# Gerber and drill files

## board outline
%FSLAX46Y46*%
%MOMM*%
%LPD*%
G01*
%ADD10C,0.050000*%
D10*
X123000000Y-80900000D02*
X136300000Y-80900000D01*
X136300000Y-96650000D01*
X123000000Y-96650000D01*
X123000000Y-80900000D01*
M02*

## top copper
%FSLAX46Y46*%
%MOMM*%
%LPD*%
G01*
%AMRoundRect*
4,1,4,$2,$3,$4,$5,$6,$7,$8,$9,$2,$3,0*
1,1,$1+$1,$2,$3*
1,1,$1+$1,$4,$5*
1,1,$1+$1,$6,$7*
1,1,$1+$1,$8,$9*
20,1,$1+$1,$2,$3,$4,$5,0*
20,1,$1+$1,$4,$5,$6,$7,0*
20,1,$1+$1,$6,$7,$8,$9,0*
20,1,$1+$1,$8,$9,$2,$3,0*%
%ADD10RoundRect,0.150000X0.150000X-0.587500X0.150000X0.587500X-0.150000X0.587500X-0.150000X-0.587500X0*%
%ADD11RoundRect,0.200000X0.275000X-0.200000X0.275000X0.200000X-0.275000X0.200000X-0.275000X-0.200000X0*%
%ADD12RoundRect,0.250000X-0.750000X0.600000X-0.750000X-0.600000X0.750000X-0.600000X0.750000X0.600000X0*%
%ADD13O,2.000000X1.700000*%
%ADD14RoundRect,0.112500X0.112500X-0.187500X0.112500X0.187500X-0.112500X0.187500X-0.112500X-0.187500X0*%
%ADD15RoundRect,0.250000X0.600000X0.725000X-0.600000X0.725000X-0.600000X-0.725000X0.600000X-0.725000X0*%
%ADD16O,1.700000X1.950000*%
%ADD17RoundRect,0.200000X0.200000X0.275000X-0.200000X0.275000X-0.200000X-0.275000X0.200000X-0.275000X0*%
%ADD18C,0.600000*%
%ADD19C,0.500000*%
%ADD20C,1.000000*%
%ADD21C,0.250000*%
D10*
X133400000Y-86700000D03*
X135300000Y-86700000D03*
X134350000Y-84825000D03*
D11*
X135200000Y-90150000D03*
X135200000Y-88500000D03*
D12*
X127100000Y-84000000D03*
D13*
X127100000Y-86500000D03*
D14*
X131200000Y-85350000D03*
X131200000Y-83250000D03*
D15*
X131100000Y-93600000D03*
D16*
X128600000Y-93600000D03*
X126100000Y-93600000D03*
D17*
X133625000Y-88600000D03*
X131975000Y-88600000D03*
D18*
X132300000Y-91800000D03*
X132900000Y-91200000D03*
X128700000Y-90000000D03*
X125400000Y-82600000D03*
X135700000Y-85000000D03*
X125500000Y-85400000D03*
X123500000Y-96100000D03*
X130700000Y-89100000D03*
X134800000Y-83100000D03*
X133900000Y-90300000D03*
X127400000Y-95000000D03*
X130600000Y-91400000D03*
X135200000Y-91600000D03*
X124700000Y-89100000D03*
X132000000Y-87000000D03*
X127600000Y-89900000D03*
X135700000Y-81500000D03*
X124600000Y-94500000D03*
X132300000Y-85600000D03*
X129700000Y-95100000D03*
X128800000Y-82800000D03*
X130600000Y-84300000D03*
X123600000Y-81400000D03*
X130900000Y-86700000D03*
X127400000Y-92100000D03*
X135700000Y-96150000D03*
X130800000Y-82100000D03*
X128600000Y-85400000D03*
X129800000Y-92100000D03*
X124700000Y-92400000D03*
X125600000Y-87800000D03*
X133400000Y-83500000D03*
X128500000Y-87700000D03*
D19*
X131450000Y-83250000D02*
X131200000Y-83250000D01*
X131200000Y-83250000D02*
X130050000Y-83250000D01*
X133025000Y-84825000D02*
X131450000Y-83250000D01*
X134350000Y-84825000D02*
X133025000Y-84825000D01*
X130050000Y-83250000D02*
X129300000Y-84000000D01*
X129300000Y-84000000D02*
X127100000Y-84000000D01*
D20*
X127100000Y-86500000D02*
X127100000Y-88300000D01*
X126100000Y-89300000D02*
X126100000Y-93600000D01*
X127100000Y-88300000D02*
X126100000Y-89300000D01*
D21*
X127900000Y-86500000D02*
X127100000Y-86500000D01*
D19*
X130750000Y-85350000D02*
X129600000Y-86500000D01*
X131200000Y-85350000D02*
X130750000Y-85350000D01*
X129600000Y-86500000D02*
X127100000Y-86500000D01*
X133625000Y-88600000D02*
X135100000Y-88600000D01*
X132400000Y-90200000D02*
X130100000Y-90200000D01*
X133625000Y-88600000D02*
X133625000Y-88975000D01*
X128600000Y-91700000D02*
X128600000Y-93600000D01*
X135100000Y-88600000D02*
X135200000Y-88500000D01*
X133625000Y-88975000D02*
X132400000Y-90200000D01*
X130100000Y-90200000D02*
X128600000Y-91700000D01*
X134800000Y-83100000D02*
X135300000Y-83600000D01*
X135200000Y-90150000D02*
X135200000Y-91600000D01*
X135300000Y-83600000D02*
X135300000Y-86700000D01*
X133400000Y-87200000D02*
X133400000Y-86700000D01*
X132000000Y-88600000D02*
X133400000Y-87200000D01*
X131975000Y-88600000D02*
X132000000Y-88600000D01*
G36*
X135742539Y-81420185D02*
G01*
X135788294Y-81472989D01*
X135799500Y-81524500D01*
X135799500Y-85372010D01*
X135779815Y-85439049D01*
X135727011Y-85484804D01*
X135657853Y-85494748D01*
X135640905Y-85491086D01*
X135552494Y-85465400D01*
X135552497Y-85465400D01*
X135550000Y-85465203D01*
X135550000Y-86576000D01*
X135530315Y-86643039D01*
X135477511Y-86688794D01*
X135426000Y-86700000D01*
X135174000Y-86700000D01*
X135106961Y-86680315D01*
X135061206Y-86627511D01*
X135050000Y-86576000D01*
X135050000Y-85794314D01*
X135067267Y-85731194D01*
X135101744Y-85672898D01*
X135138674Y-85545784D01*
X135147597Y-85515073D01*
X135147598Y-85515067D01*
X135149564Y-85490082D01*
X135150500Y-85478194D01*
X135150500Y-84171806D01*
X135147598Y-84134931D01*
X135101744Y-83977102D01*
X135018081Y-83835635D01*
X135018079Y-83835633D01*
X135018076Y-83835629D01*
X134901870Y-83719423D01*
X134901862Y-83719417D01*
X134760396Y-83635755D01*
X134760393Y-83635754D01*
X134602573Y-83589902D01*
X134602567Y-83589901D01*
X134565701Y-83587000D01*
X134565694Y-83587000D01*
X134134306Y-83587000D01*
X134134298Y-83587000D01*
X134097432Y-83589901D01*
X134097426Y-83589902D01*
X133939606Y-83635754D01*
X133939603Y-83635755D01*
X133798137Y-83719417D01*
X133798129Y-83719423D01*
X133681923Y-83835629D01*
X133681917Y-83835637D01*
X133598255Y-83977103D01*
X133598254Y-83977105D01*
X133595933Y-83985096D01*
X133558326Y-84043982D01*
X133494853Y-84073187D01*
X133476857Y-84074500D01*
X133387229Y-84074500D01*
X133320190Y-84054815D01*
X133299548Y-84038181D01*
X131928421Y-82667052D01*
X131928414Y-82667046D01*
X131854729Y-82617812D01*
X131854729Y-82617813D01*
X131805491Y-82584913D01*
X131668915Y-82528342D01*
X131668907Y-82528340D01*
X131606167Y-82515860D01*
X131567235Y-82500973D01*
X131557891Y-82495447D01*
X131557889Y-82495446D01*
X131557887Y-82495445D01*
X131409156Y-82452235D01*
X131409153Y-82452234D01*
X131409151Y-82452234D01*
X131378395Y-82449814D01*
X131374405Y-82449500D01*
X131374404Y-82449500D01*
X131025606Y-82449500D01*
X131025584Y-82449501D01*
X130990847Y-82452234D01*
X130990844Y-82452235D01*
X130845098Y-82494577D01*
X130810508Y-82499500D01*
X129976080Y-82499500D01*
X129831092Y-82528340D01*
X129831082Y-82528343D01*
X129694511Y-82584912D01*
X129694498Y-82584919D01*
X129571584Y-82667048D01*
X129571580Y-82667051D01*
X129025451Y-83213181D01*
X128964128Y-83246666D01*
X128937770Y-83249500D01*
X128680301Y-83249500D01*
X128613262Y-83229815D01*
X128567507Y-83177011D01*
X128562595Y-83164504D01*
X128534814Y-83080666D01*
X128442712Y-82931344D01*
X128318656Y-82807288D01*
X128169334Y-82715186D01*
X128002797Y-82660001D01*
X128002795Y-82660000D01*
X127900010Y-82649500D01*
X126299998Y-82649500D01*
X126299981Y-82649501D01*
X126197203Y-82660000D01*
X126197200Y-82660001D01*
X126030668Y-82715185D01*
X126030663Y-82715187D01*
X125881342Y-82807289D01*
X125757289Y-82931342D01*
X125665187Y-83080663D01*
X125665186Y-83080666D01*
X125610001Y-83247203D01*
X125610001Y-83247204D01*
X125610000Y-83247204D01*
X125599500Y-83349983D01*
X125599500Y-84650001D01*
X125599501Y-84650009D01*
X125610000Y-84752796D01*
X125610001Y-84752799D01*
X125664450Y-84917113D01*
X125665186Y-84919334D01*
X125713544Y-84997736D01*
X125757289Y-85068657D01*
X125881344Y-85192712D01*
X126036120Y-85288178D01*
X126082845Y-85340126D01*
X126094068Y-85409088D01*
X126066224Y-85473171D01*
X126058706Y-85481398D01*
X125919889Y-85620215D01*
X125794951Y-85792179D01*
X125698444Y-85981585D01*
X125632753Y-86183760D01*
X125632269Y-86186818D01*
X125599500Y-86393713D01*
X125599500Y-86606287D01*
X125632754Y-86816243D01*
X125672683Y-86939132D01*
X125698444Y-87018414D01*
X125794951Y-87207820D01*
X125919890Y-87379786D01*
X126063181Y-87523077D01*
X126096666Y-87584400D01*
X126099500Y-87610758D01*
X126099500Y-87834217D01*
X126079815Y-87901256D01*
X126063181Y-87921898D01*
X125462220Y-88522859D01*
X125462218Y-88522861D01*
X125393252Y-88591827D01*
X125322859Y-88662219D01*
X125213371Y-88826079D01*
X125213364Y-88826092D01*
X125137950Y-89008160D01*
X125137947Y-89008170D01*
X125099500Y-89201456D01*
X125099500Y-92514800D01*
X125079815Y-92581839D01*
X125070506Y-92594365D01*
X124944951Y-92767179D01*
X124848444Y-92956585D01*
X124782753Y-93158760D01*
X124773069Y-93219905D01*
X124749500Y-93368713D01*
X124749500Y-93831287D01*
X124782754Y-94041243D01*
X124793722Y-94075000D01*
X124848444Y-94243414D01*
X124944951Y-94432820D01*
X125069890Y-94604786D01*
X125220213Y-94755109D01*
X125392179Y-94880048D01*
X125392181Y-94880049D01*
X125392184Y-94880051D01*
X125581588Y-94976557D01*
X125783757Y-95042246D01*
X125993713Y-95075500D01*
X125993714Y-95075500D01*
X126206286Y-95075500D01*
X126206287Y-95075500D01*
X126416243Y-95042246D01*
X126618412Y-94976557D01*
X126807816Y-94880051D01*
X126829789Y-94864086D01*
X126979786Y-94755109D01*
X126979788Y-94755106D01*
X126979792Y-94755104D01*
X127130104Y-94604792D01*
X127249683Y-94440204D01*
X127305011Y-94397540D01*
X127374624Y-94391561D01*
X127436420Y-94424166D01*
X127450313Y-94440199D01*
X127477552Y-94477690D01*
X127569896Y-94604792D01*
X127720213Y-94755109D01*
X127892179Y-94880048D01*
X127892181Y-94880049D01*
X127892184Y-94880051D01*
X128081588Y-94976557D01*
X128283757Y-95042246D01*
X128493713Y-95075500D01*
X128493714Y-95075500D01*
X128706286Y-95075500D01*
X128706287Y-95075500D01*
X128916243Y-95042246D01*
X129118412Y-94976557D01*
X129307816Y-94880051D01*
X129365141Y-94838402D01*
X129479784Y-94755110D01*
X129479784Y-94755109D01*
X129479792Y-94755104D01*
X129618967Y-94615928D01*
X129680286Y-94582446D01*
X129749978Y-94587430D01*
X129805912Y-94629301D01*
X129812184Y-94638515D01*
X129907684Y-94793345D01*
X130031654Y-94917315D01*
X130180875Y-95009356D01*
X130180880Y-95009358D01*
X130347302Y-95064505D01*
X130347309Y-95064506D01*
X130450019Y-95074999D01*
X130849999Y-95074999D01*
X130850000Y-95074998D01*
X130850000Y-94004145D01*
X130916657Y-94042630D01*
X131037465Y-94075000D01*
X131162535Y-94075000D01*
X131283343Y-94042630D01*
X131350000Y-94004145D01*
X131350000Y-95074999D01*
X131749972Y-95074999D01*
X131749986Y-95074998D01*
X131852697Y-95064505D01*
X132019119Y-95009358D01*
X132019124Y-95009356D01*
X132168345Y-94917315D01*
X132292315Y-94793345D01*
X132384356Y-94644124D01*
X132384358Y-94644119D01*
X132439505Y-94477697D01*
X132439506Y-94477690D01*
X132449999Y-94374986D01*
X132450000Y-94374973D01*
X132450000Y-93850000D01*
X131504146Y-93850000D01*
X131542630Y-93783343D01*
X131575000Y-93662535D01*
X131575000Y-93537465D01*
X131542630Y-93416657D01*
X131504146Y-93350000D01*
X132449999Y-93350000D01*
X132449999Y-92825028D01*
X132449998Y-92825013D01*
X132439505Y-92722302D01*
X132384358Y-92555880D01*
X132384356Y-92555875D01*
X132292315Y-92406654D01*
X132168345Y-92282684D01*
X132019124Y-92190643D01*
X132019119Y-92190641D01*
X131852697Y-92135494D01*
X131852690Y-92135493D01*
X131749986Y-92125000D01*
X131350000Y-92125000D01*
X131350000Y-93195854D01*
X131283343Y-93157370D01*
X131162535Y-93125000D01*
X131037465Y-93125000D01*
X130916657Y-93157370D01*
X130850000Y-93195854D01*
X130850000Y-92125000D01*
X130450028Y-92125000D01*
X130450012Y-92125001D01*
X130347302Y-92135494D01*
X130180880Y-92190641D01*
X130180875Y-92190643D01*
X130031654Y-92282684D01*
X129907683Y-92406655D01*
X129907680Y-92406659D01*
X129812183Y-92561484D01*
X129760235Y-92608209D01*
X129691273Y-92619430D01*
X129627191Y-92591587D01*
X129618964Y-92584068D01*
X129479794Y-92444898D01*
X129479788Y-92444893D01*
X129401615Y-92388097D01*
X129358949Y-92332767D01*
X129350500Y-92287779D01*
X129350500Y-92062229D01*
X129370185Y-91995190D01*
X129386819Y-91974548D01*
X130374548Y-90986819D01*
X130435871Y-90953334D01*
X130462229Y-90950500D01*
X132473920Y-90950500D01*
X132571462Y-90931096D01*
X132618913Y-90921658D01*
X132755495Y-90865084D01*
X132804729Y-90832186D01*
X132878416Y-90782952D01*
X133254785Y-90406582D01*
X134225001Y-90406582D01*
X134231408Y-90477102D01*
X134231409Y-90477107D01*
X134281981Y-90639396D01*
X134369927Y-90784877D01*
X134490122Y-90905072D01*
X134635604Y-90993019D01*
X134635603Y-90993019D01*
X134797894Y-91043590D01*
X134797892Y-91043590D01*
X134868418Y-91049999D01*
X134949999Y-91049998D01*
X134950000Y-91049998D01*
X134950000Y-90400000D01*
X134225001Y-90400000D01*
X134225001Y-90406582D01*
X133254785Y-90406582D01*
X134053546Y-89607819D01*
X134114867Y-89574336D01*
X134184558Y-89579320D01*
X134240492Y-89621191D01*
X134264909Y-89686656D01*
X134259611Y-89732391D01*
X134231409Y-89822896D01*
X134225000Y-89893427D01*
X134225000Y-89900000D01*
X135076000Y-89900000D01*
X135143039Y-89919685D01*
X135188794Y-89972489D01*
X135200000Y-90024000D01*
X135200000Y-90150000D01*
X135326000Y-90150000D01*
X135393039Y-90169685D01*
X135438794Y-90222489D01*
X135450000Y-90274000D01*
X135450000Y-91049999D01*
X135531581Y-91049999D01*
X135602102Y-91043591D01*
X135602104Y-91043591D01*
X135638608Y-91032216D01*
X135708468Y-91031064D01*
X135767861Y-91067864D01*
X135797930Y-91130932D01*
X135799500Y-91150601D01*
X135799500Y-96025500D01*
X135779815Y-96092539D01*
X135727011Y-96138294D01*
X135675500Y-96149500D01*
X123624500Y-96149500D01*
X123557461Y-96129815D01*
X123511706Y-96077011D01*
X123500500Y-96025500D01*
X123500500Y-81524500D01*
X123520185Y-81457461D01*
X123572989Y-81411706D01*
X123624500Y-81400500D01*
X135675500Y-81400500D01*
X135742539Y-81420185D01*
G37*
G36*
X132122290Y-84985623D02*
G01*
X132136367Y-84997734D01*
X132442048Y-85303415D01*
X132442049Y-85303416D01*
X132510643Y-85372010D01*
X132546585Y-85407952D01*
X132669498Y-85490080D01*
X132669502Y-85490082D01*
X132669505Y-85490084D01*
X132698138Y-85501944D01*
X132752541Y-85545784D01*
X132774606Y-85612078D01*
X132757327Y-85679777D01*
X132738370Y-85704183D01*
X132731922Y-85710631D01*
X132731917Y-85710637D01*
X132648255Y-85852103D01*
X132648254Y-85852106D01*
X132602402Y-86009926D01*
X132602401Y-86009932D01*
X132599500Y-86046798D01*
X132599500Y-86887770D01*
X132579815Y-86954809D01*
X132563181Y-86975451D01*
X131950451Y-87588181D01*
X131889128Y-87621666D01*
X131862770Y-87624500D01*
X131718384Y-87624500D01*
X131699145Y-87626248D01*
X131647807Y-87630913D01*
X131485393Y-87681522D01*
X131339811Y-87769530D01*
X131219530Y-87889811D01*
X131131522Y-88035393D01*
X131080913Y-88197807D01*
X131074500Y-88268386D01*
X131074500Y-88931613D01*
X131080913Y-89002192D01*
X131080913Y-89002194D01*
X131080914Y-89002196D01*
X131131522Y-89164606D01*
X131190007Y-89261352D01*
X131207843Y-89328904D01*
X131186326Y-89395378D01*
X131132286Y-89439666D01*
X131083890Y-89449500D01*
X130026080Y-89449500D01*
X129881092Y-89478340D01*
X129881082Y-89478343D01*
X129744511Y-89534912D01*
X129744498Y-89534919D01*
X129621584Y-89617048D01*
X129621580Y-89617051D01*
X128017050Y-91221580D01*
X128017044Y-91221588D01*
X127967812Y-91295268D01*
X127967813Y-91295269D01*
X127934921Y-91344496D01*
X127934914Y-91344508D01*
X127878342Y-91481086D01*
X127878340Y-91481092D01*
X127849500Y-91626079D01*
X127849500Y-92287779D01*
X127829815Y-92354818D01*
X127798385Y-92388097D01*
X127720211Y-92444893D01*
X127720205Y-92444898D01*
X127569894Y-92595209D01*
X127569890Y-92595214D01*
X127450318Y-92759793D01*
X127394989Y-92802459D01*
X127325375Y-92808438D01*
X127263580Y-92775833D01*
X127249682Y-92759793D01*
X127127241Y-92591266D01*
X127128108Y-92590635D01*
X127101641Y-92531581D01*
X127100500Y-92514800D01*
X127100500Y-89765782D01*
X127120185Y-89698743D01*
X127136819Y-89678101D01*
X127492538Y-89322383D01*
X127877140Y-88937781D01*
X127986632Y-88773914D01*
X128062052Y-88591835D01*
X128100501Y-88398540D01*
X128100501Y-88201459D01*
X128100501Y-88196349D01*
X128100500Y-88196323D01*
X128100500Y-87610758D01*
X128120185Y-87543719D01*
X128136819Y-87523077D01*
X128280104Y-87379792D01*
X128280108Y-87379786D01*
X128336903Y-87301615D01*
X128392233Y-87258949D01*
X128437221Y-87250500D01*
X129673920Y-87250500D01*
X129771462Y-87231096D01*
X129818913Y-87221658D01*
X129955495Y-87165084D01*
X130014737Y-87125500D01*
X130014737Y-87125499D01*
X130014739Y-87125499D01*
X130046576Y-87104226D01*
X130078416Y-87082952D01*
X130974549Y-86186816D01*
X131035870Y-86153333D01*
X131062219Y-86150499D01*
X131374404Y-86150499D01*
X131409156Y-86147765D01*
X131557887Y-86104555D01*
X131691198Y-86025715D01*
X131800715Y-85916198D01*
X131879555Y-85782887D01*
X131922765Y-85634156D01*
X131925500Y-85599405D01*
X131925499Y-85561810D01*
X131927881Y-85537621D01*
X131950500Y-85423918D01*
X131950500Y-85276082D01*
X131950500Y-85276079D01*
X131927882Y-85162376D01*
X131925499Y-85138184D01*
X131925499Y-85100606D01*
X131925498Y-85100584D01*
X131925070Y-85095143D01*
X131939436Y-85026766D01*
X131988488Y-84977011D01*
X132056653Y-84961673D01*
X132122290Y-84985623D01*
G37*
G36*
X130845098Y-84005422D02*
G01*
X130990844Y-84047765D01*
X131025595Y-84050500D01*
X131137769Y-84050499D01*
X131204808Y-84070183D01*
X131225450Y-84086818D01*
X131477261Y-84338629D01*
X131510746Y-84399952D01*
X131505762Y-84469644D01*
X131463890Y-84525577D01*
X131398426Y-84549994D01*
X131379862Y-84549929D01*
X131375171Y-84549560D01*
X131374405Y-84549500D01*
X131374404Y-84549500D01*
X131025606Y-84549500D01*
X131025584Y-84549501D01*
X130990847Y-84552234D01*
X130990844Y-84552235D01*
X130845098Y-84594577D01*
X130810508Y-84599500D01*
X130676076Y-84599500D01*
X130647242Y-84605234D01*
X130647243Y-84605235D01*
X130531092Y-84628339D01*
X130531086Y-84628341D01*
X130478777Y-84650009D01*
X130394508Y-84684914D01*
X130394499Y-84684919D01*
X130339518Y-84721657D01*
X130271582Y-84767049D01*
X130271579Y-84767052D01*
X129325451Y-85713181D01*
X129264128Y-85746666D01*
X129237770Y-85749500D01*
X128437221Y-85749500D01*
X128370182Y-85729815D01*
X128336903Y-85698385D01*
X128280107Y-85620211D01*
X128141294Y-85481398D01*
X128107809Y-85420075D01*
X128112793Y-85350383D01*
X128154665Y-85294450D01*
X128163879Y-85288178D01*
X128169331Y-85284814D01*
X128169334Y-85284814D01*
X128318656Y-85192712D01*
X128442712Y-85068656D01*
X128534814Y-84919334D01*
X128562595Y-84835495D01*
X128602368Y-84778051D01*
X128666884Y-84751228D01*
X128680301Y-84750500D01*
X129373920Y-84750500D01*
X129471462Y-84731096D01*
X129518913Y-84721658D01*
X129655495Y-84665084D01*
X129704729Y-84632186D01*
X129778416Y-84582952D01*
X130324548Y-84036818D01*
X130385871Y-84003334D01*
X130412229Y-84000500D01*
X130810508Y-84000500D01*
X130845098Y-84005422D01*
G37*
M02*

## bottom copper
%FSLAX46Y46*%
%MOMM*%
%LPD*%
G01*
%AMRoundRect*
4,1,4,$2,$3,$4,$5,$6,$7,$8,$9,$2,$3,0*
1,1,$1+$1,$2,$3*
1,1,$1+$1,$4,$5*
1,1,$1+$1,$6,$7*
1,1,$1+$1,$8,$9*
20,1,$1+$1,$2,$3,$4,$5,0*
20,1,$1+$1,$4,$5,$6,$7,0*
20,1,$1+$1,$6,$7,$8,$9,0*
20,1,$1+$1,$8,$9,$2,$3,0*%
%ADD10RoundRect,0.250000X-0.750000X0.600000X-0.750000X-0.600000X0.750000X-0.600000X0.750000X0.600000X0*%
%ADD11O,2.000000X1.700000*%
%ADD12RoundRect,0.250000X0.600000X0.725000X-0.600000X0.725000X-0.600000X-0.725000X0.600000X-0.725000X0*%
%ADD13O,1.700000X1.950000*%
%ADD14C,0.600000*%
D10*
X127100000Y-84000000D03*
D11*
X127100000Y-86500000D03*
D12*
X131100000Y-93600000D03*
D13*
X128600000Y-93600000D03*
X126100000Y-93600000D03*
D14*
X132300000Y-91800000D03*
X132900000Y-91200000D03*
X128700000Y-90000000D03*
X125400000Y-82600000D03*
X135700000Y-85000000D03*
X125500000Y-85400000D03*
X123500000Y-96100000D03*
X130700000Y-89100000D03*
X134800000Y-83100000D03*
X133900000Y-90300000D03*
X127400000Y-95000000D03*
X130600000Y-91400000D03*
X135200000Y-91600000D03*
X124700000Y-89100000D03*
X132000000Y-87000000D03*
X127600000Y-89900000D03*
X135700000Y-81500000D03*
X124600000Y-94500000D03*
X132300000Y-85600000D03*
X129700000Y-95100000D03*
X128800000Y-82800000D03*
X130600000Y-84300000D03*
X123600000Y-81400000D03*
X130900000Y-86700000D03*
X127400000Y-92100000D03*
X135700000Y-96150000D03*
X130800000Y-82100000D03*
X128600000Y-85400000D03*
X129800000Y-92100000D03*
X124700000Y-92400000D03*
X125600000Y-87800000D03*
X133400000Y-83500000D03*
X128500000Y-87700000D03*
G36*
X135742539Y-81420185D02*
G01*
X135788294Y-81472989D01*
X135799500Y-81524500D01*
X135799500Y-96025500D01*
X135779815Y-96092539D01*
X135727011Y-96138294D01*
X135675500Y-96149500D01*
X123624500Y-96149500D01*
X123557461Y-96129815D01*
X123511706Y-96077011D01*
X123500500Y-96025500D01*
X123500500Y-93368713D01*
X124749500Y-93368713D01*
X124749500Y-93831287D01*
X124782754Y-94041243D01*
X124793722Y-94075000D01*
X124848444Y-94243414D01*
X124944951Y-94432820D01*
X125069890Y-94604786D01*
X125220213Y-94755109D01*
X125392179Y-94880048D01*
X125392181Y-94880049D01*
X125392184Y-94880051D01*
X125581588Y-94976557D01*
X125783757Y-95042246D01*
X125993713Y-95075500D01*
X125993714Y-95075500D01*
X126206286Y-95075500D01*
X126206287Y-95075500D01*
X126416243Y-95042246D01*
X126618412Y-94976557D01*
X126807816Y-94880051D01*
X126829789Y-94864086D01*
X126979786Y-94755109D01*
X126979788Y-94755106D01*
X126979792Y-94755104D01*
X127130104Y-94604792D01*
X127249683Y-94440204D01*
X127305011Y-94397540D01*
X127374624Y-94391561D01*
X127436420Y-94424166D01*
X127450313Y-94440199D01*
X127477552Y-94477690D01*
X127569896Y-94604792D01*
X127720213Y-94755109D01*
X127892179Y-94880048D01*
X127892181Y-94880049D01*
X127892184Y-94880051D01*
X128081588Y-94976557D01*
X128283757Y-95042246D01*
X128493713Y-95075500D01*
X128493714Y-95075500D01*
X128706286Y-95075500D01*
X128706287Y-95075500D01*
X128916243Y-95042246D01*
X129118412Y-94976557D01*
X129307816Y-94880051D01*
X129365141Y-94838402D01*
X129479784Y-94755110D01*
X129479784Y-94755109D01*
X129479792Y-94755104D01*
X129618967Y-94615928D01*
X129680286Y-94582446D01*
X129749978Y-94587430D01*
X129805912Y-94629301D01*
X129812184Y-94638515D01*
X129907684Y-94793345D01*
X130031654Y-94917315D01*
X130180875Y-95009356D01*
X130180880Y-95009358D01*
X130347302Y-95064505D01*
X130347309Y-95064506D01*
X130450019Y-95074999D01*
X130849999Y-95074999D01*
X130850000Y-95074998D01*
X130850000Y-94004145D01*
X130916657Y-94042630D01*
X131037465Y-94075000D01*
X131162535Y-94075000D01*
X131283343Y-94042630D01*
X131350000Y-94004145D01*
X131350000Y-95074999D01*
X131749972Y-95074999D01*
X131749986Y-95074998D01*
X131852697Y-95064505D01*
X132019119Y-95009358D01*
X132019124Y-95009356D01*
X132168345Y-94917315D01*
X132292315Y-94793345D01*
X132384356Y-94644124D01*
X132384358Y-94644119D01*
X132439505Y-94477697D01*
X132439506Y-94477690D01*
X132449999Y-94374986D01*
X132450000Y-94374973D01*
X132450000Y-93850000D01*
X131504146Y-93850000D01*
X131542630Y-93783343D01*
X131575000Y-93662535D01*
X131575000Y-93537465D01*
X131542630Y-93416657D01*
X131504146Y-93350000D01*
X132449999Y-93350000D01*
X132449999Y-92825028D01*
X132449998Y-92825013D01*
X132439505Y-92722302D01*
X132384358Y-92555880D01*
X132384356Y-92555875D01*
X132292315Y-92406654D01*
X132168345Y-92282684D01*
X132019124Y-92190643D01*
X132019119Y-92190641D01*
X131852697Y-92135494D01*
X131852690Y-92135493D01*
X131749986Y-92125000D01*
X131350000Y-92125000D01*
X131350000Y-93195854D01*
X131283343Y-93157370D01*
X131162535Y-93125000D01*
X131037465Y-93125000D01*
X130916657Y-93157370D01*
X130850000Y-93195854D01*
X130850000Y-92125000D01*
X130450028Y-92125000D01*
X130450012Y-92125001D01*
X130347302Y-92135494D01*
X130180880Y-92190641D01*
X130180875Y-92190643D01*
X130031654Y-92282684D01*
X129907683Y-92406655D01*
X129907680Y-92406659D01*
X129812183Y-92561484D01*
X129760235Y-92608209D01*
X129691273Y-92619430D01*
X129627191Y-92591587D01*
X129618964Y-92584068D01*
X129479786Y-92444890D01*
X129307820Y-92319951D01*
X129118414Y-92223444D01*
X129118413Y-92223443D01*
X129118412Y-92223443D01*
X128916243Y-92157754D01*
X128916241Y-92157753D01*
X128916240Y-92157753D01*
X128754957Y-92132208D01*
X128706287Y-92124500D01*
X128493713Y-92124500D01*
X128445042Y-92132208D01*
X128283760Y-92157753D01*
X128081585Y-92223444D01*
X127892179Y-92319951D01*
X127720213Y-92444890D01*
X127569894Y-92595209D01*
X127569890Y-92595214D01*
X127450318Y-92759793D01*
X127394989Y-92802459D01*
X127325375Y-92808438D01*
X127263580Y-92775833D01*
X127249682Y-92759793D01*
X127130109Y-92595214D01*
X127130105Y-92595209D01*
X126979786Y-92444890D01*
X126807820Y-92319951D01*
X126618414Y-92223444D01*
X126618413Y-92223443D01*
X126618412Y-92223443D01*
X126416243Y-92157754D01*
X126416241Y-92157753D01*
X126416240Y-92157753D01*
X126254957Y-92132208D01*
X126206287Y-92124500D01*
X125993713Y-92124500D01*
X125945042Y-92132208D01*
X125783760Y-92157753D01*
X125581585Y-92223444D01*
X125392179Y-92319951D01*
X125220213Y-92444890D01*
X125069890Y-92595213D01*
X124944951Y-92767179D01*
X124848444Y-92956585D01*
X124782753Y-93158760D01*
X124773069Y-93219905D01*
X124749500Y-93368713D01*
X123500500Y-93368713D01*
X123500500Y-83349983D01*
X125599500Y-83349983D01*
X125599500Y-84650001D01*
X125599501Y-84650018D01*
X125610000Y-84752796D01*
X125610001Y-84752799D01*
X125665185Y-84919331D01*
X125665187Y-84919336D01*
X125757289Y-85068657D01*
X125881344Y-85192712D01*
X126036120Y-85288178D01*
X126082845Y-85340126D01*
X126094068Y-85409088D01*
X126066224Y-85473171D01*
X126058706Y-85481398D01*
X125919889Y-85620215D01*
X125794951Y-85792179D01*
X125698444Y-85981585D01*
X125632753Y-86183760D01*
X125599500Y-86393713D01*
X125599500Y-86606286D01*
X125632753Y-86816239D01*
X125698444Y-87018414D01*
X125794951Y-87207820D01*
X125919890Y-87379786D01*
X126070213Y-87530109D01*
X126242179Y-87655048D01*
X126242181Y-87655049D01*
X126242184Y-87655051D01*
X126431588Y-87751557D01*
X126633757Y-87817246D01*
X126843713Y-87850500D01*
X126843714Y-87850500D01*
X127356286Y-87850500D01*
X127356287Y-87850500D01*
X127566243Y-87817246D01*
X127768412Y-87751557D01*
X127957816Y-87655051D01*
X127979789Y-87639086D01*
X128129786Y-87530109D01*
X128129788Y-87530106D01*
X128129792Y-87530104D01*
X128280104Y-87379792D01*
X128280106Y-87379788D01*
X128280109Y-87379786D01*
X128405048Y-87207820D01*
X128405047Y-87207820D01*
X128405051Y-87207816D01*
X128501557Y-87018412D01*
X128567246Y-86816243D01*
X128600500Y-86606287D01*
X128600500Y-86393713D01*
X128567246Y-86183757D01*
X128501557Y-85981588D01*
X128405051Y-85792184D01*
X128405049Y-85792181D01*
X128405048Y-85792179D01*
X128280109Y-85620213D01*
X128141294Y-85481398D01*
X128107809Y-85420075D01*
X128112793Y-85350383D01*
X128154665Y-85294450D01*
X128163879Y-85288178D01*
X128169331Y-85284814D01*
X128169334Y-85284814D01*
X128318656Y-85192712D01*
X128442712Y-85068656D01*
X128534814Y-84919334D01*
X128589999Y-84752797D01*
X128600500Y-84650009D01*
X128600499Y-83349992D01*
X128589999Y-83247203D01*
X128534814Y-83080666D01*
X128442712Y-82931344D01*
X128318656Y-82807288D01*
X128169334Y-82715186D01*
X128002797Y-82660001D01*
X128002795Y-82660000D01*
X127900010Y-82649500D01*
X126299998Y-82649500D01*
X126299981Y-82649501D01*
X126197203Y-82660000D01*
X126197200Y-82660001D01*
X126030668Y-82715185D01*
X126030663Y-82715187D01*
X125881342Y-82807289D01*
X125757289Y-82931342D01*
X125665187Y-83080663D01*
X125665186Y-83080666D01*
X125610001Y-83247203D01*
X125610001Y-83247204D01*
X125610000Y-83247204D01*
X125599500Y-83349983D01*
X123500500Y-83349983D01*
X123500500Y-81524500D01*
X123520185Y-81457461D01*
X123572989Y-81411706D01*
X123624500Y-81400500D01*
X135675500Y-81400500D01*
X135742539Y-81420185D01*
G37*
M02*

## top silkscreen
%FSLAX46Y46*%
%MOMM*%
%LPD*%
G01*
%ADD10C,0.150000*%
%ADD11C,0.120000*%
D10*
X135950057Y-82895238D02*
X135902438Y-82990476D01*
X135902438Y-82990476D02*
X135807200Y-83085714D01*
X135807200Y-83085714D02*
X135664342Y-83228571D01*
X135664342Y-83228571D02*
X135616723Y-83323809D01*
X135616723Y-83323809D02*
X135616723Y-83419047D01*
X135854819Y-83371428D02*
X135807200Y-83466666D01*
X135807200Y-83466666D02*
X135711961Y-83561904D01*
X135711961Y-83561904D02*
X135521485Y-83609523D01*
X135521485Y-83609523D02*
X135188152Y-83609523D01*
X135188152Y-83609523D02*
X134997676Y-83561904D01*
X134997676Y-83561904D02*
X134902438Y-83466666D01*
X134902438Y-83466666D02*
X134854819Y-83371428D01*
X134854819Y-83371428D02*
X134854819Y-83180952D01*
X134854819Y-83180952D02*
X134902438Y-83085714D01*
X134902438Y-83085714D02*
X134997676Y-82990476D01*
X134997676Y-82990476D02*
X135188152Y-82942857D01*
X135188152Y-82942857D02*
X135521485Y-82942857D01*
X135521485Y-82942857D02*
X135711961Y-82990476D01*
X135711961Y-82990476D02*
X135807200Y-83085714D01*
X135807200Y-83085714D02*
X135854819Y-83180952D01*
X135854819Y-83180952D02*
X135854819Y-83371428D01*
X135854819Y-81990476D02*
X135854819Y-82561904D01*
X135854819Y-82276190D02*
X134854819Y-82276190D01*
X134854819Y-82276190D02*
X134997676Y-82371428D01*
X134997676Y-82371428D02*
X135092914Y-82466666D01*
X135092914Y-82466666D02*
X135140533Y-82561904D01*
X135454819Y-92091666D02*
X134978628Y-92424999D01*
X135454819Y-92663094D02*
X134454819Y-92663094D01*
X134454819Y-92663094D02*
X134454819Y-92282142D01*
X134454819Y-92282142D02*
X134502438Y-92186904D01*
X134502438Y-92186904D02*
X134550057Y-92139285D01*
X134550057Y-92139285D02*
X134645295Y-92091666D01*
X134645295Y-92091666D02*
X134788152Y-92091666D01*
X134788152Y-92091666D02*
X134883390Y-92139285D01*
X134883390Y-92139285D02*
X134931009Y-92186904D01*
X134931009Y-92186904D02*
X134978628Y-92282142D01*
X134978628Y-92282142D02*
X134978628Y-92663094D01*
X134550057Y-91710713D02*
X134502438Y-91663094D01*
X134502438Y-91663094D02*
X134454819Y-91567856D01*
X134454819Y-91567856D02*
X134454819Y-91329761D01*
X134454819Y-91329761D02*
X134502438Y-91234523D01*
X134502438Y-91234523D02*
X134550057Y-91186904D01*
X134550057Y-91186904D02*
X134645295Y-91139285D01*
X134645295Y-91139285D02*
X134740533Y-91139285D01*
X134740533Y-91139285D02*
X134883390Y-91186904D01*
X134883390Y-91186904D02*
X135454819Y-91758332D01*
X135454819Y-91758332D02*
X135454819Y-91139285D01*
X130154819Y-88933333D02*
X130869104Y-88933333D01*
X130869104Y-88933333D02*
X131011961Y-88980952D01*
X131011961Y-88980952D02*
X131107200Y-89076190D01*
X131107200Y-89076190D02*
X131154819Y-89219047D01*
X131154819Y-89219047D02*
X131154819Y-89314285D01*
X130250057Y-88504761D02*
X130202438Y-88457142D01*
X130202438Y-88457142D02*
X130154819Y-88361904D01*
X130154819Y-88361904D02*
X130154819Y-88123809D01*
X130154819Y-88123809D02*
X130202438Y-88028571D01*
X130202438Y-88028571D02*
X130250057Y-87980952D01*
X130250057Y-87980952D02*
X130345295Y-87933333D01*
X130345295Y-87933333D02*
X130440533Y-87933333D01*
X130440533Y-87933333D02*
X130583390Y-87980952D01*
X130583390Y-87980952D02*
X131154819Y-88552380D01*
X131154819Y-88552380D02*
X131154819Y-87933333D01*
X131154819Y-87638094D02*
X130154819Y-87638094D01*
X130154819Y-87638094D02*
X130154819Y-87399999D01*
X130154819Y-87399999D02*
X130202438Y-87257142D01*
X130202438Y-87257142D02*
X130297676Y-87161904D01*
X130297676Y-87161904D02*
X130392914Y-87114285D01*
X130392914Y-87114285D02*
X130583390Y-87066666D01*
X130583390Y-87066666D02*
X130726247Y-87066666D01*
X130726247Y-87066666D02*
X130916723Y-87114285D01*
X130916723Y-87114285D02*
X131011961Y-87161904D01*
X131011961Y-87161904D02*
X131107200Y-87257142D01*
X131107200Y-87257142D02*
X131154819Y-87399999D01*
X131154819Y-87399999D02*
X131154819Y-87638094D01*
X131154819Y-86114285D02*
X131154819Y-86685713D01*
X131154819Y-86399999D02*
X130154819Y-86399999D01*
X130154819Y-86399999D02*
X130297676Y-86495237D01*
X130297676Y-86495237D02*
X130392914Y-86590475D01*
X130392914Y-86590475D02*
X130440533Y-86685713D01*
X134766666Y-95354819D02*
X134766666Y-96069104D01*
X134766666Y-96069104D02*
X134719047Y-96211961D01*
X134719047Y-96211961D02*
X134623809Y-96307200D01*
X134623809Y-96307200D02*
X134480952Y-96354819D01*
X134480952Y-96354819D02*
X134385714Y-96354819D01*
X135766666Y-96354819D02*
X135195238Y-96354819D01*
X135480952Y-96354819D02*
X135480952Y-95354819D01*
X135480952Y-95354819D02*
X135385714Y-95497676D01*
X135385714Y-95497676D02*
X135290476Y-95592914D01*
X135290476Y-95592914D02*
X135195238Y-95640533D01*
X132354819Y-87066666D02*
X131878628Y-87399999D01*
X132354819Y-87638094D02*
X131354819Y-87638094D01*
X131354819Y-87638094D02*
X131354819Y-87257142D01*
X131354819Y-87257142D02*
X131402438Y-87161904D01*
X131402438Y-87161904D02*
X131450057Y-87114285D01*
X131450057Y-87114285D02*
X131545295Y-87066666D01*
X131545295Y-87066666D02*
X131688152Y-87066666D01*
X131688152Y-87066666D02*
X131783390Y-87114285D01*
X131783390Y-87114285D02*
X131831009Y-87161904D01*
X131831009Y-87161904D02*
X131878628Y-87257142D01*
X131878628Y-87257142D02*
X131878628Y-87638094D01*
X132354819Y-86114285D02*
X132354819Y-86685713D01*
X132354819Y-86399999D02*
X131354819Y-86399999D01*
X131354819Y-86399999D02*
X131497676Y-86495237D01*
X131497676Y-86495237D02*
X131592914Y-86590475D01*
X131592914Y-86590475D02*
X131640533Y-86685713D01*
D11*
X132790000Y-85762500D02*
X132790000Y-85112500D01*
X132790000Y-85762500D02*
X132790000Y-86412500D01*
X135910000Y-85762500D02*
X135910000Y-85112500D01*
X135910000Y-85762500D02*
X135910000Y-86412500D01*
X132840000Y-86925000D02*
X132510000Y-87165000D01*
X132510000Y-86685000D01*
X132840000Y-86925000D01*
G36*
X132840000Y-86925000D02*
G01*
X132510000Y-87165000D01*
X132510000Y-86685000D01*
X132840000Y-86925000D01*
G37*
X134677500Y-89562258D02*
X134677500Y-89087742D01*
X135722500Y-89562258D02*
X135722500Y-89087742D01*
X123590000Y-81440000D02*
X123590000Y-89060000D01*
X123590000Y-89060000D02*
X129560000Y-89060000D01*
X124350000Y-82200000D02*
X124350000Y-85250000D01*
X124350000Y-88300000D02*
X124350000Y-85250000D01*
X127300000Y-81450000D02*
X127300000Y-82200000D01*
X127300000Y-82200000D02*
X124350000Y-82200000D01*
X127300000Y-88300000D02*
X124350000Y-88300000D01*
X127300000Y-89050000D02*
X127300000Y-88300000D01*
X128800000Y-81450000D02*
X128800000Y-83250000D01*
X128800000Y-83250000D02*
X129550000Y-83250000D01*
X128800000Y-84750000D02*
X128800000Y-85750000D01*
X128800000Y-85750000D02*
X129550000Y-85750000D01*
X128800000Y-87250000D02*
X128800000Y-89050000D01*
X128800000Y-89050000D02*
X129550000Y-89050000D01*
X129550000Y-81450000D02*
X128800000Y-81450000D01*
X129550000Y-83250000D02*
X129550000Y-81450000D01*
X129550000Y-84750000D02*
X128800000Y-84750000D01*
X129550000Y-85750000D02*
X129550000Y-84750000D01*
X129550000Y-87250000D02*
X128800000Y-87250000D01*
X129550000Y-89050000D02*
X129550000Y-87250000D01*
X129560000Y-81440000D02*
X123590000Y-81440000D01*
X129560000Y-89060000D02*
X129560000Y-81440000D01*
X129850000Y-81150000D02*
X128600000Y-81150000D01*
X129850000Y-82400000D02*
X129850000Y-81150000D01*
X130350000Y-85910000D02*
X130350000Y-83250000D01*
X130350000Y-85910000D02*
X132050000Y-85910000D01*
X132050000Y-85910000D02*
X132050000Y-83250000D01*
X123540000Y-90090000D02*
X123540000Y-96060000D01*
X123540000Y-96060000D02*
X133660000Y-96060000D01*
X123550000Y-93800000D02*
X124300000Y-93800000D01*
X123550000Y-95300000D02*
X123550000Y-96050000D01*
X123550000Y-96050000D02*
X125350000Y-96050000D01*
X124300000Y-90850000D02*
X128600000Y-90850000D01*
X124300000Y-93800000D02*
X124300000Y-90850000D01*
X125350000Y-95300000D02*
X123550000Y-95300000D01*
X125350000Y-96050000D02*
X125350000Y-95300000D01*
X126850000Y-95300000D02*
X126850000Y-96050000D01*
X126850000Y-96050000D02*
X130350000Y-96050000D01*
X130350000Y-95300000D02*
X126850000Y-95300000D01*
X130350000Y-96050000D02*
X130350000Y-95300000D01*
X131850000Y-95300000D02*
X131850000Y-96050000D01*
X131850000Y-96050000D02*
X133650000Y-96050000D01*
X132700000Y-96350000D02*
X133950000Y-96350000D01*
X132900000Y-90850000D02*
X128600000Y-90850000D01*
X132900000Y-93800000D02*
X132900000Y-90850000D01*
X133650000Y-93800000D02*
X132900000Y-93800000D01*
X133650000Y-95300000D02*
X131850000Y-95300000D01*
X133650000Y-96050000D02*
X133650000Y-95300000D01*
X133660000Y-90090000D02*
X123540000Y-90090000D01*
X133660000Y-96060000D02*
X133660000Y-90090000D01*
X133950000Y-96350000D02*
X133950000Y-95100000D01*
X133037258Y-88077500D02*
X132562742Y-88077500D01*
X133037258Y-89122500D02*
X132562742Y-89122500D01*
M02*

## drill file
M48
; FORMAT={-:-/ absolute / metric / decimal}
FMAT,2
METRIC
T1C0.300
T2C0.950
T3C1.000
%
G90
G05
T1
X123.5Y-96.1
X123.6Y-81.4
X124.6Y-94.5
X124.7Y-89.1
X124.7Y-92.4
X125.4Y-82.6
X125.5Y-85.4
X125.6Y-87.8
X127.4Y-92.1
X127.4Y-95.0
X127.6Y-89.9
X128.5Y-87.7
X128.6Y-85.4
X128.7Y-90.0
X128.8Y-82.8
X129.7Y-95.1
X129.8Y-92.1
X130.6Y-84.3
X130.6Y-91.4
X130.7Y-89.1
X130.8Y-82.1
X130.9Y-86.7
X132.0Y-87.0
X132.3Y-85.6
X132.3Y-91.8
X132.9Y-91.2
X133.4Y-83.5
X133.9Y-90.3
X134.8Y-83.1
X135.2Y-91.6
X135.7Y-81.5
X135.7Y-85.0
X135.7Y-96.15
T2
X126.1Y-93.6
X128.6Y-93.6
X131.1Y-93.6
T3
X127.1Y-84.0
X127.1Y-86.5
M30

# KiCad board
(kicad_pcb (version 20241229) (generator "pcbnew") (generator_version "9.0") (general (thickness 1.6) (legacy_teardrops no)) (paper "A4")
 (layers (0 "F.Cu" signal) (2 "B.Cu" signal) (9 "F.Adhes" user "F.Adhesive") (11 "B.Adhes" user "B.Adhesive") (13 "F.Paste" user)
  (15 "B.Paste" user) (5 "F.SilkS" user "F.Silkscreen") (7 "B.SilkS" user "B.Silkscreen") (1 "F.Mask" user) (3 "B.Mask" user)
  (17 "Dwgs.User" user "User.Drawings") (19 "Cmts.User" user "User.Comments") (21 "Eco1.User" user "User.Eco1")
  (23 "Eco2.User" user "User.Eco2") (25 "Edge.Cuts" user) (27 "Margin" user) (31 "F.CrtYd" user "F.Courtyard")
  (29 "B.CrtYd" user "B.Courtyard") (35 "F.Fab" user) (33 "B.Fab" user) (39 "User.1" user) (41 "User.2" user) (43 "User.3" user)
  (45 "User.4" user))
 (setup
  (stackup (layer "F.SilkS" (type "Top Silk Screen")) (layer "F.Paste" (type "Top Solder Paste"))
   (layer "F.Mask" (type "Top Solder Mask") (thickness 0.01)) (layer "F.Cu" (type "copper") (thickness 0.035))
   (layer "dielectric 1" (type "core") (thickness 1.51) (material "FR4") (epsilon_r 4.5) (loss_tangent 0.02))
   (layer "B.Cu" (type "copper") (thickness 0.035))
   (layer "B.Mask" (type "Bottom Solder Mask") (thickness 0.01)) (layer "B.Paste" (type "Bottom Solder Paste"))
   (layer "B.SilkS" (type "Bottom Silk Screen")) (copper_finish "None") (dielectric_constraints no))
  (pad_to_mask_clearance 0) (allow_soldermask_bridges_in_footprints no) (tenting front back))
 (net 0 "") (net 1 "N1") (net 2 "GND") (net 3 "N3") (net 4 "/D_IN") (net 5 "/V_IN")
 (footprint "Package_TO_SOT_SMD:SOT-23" (layer "F.Cu") (at 134.35 85.7625 90)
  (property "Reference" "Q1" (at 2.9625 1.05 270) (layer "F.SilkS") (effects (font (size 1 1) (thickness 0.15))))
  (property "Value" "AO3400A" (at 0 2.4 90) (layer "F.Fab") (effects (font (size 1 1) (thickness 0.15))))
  (fp_line (start 0 -1.56) (end 0.65 -1.56) (stroke (width 0.12) (type solid)) (layer "F.SilkS"))
  (fp_line (start 0 -1.56) (end -0.65 -1.56) (stroke (width 0.12) (type solid)) (layer "F.SilkS"))
  (fp_line (start 0 1.56) (end 0.65 1.56) (stroke (width 0.12) (type solid)) (layer "F.SilkS"))
  (fp_line (start 0 1.56) (end -0.65 1.56) (stroke (width 0.12) (type solid)) (layer "F.SilkS"))
  (fp_poly (pts (xy -1.1625 -1.51) (xy -1.4025 -1.84) (xy -0.9225 -1.84)) (stroke (width 0.12) (type solid)) (fill yes) (layer "F.SilkS"))
  (pad "1" smd roundrect (at -0.9375 -0.95 90) (size 1.475 0.6) (layers "F.Cu" "F.Mask" "F.Paste") (roundrect_rratio 0.25) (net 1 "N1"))
  (pad "2" smd roundrect (at -0.9375 0.95 90) (size 1.475 0.6) (layers "F.Cu" "F.Mask" "F.Paste") (roundrect_rratio 0.25) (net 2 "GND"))
  (pad "3" smd roundrect (at 0.9375 0 90) (size 1.475 0.6) (layers "F.Cu" "F.Mask" "F.Paste") (roundrect_rratio 0.25) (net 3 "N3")))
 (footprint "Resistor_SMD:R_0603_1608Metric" (layer "F.Cu") (at 135.2 89.325 90)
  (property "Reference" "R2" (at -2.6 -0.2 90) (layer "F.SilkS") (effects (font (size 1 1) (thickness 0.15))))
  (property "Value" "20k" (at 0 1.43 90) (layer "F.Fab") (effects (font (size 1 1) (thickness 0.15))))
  (fp_line (start -0.237258 -0.5225) (end 0.237258 -0.5225) (stroke (width 0.12) (type solid)) (layer "F.SilkS"))
  (fp_line (start -0.237258 0.5225) (end 0.237258 0.5225) (stroke (width 0.12) (type solid)) (layer "F.SilkS"))
  (pad "1" smd roundrect (at -0.825 0 90) (size 0.8 0.95) (layers "F.Cu" "F.Mask" "F.Paste") (roundrect_rratio 0.25) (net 2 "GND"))
  (pad "2" smd roundrect (at 0.825 0 90) (size 0.8 0.95) (layers "F.Cu" "F.Mask" "F.Paste") (roundrect_rratio 0.25) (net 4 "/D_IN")))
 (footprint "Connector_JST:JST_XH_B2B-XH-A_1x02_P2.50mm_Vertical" (layer "F.Cu") (at 127.1 84 -90)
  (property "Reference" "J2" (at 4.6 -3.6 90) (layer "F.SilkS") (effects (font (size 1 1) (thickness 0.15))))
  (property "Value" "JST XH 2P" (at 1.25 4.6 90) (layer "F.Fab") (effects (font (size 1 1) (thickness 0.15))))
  (fp_line (start -2.56 3.51) (end 5.06 3.51) (stroke (width 0.12) (type solid)) (layer "F.SilkS"))
  (fp_line (start 5.06 3.51) (end 5.06 -2.46) (stroke (width 0.12) (type solid)) (layer "F.SilkS"))
  (fp_line (start -1.8 2.75) (end 1.25 2.75) (stroke (width 0.12) (type solid)) (layer "F.SilkS"))
  (fp_line (start 4.3 2.75) (end 1.25 2.75) (stroke (width 0.12) (type solid)) (layer "F.SilkS"))
  (fp_line (start -2.55 -0.2) (end -1.8 -0.2) (stroke (width 0.12) (type solid)) (layer "F.SilkS"))
  (fp_line (start -1.8 -0.2) (end -1.8 2.75) (stroke (width 0.12) (type solid)) (layer "F.SilkS"))
  (fp_line (start 4.3 -0.2) (end 4.3 2.75) (stroke (width 0.12) (type solid)) (layer "F.SilkS"))
  (fp_line (start 5.05 -0.2) (end 4.3 -0.2) (stroke (width 0.12) (type solid)) (layer "F.SilkS"))
  (fp_line (start -2.55 -1.7) (end -0.75 -1.7) (stroke (width 0.12) (type solid)) (layer "F.SilkS"))
  (fp_line (start -0.75 -1.7) (end -0.75 -2.45) (stroke (width 0.12) (type solid)) (layer "F.SilkS"))
  (fp_line (start 0.75 -1.7) (end 1.75 -1.7) (stroke (width 0.12) (type solid)) (layer "F.SilkS"))
  (fp_line (start 1.75 -1.7) (end 1.75 -2.45) (stroke (width 0.12) (type solid)) (layer "F.SilkS"))
  (fp_line (start 3.25 -1.7) (end 5.05 -1.7) (stroke (width 0.12) (type solid)) (layer "F.SilkS"))
  (fp_line (start 5.05 -1.7) (end 5.05 -2.45) (stroke (width 0.12) (type solid)) (layer "F.SilkS"))
  (fp_line (start -2.55 -2.45) (end -2.55 -1.7) (stroke (width 0.12) (type solid)) (layer "F.SilkS"))
  (fp_line (start -0.75 -2.45) (end -2.55 -2.45) (stroke (width 0.12) (type solid)) (layer "F.SilkS"))
  (fp_line (start 0.75 -2.45) (end 0.75 -1.7) (stroke (width 0.12) (type solid)) (layer "F.SilkS"))
  (fp_line (start 1.75 -2.45) (end 0.75 -2.45) (stroke (width 0.12) (type solid)) (layer "F.SilkS"))
  (fp_line (start 3.25 -2.45) (end 3.25 -1.7) (stroke (width 0.12) (type solid)) (layer "F.SilkS"))
  (fp_line (start 5.05 -2.45) (end 3.25 -2.45) (stroke (width 0.12) (type solid)) (layer "F.SilkS"))
  (fp_line (start -2.56 -2.46) (end -2.56 3.51) (stroke (width 0.12) (type solid)) (layer "F.SilkS"))
  (fp_line (start 5.06 -2.46) (end -2.56 -2.46) (stroke (width 0.12) (type solid)) (layer "F.SilkS"))
  (fp_line (start -2.85 -2.75) (end -2.85 -1.5) (stroke (width 0.12) (type solid)) (layer "F.SilkS"))
  (fp_line (start -1.6 -2.75) (end -2.85 -2.75) (stroke (width 0.12) (type solid)) (layer "F.SilkS"))
  (pad "1" thru_hole roundrect (at 0 0 270) (size 1.7 2) (drill 1) (layers "*.Cu" "*.Mask") (remove_unused_layers no)
   (roundrect_rratio 0.147059) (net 3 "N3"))
  (pad "2" thru_hole oval (at 2.5 0 270) (size 1.7 2) (drill 1) (layers "*.Cu" "*.Mask") (remove_unused_layers no) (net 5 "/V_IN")))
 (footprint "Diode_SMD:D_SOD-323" (layer "F.Cu") (at 131.2 84.3 90)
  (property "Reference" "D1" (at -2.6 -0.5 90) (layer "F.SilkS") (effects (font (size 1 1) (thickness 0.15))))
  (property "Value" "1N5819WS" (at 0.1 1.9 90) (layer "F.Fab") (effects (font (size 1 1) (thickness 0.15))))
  (fp_line (start -1.61 -0.85) (end 1.05 -0.85) (stroke (width 0.12) (type solid)) (layer "F.SilkS"))
  (fp_line (start -1.61 -0.85) (end -1.61 0.85) (stroke (width 0.12) (type solid)) (layer "F.SilkS"))
  (fp_line (start -1.61 0.85) (end 1.05 0.85) (stroke (width 0.12) (type solid)) (layer "F.SilkS"))
  (pad "1" smd roundrect (at -1.05 0 90) (size 0.6 0.45) (layers "F.Cu" "F.Mask" "F.Paste") (roundrect_rratio 0.25) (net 5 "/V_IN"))
  (pad "2" smd roundrect (at 1.05 0 90) (size 0.6 0.45) (layers "F.Cu" "F.Mask" "F.Paste") (roundrect_rratio 0.25) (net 3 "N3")))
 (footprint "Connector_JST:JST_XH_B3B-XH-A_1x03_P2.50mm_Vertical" (layer "F.Cu") (at 131.1 93.6 180)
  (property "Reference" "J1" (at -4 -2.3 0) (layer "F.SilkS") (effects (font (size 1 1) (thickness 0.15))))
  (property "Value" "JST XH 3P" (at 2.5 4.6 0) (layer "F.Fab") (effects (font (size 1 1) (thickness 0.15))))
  (fp_line (start 7.56 3.51) (end 7.56 -2.46) (stroke (width 0.12) (type solid)) (layer "F.SilkS"))
  (fp_line (start 7.56 -2.46) (end -2.56 -2.46) (stroke (width 0.12) (type solid)) (layer "F.SilkS"))
  (fp_line (start 7.55 -0.2) (end 6.8 -0.2) (stroke (width 0.12) (type solid)) (layer "F.SilkS"))
  (fp_line (start 7.55 -1.7) (end 7.55 -2.45) (stroke (width 0.12) (type solid)) (layer "F.SilkS"))
  (fp_line (start 7.55 -2.45) (end 5.75 -2.45) (stroke (width 0.12) (type solid)) (layer "F.SilkS"))
  (fp_line (start 6.8 2.75) (end 2.5 2.75) (stroke (width 0.12) (type solid)) (layer "F.SilkS"))
  (fp_line (start 6.8 -0.2) (end 6.8 2.75) (stroke (width 0.12) (type solid)) (layer "F.SilkS"))
  (fp_line (start 5.75 -1.7) (end 7.55 -1.7) (stroke (width 0.12) (type solid)) (layer "F.SilkS"))
  (fp_line (start 5.75 -2.45) (end 5.75 -1.7) (stroke (width 0.12) (type solid)) (layer "F.SilkS"))
  (fp_line (start 4.25 -1.7) (end 4.25 -2.45) (stroke (width 0.12) (type solid)) (layer "F.SilkS"))
  (fp_line (start 4.25 -2.45) (end 0.75 -2.45) (stroke (width 0.12) (type solid)) (layer "F.SilkS"))
  (fp_line (start 0.75 -1.7) (end 4.25 -1.7) (stroke (width 0.12) (type solid)) (layer "F.SilkS"))
  (fp_line (start 0.75 -2.45) (end 0.75 -1.7) (stroke (width 0.12) (type solid)) (layer "F.SilkS"))
  (fp_line (start -0.75 -1.7) (end -0.75 -2.45) (stroke (width 0.12) (type solid)) (layer "F.SilkS"))
  (fp_line (start -0.75 -2.45) (end -2.55 -2.45) (stroke (width 0.12) (type solid)) (layer "F.SilkS"))
  (fp_line (start -1.6 -2.75) (end -2.85 -2.75) (stroke (width 0.12) (type solid)) (layer "F.SilkS"))
  (fp_line (start -1.8 2.75) (end 2.5 2.75) (stroke (width 0.12) (type solid)) (layer "F.SilkS"))
  (fp_line (start -1.8 -0.2) (end -1.8 2.75) (stroke (width 0.12) (type solid)) (layer "F.SilkS"))
  (fp_line (start -2.55 -0.2) (end -1.8 -0.2) (stroke (width 0.12) (type solid)) (layer "F.SilkS"))
  (fp_line (start -2.55 -1.7) (end -0.75 -1.7) (stroke (width 0.12) (type solid)) (layer "F.SilkS"))
  (fp_line (start -2.55 -2.45) (end -2.55 -1.7) (stroke (width 0.12) (type solid)) (layer "F.SilkS"))
  (fp_line (start -2.56 3.51) (end 7.56 3.51) (stroke (width 0.12) (type solid)) (layer "F.SilkS"))
  (fp_line (start -2.56 -2.46) (end -2.56 3.51) (stroke (width 0.12) (type solid)) (layer "F.SilkS"))
  (fp_line (start -2.85 -2.75) (end -2.85 -1.5) (stroke (width 0.12) (type solid)) (layer "F.SilkS"))
  (pad "1" thru_hole roundrect (at 0 0 180) (size 1.7 1.95) (drill 0.95) (layers "*.Cu" "*.Mask") (remove_unused_layers no)
   (roundrect_rratio 0.147059) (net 2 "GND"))
  (pad "2" thru_hole oval (at 2.5 0 180) (size 1.7 1.95) (drill 0.95) (layers "*.Cu" "*.Mask") (remove_unused_layers no) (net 4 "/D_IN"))
  (pad "3" thru_hole oval (at 5 0 180) (size 1.7 1.95) (drill 0.95) (layers "*.Cu" "*.Mask") (remove_unused_layers no) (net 5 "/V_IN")))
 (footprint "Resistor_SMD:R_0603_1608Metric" (layer "F.Cu") (at 132.8 88.6 180)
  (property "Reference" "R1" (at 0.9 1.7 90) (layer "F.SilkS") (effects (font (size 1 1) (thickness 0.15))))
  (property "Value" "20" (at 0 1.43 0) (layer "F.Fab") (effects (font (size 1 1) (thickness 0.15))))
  (fp_line (start -0.237258 0.5225) (end 0.237258 0.5225) (stroke (width 0.12) (type solid)) (layer "F.SilkS"))
  (fp_line (start -0.237258 -0.5225) (end 0.237258 -0.5225) (stroke (width 0.12) (type solid)) (layer "F.SilkS"))
  (pad "1" smd roundrect (at -0.825 0 180) (size 0.8 0.95) (layers "F.Cu" "F.Mask" "F.Paste") (roundrect_rratio 0.25) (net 4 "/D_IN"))
  (pad "2" smd roundrect (at 0.825 0 180) (size 0.8 0.95) (layers "F.Cu" "F.Mask" "F.Paste") (roundrect_rratio 0.25) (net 1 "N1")))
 (gr_rect (start 123 80.9) (end 136.3 96.65) (stroke (width 0.05) (type default)) (fill no) (layer "Edge.Cuts"))
 (segment (start 131.45 83.25) (end 131.2 83.25) (width 0.5) (layer "F.Cu") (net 3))
 (segment (start 131.2 83.25) (end 130.05 83.25) (width 0.5) (layer "F.Cu") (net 3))
 (segment (start 133.025 84.825) (end 131.45 83.25) (width 0.5) (layer "F.Cu") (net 3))
 (segment (start 134.35 84.825) (end 133.025 84.825) (width 0.5) (layer "F.Cu") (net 3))
 (segment (start 130.05 83.25) (end 129.3 84) (width 0.5) (layer "F.Cu") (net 3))
 (segment (start 129.3 84) (end 127.1 84) (width 0.5) (layer "F.Cu") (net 3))
 (segment (start 127.1 86.5) (end 127.1 88.3) (width 1) (layer "F.Cu") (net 5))
 (segment (start 126.1 89.3) (end 126.1 93.6) (width 1) (layer "F.Cu") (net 5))
 (segment (start 127.1 88.3) (end 126.1 89.3) (width 1) (layer "F.Cu") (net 5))
 (segment (start 127.9 86.5) (end 127.1 86.5) (width 0.25) (layer "F.Cu") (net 5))
 (segment (start 130.75 85.35) (end 129.6 86.5) (width 0.5) (layer "F.Cu") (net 5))
 (segment (start 131.2 85.35) (end 130.75 85.35) (width 0.5) (layer "F.Cu") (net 5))
 (segment (start 129.6 86.5) (end 127.1 86.5) (width 0.5) (layer "F.Cu") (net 5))
 (segment (start 133.625 88.6) (end 135.1 88.6) (width 0.5) (layer "F.Cu") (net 4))
 (segment (start 132.4 90.2) (end 130.1 90.2) (width 0.5) (layer "F.Cu") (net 4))
 (segment (start 133.625 88.6) (end 133.625 88.975) (width 0.5) (layer "F.Cu") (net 4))
 (segment (start 128.6 91.7) (end 128.6 93.6) (width 0.5) (layer "F.Cu") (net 4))
 (segment (start 135.1 88.6) (end 135.2 88.5) (width 0.5) (layer "F.Cu") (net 4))
 (segment (start 133.625 88.975) (end 132.4 90.2) (width 0.5) (layer "F.Cu") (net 4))
 (segment (start 130.1 90.2) (end 128.6 91.7) (width 0.5) (layer "F.Cu") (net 4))
 (segment (start 134.8 83.1) (end 135.3 83.6) (width 0.5) (layer "F.Cu") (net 2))
 (segment (start 135.2 90.15) (end 135.2 91.6) (width 0.5) (layer "F.Cu") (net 2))
 (segment (start 135.3 83.6) (end 135.3 86.7) (width 0.5) (layer "F.Cu") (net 2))
 (via (at 132.3 91.8) (size 0.6) (drill 0.3) (layers "F.Cu" "B.Cu") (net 2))
 (via (at 132.9 91.2) (size 0.6) (drill 0.3) (layers "F.Cu" "B.Cu") (free yes) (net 2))
 (via (at 128.7 90) (size 0.6) (drill 0.3) (layers "F.Cu" "B.Cu") (free yes) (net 2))
 (via (at 125.4 82.6) (size 0.6) (drill 0.3) (layers "F.Cu" "B.Cu") (free yes) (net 2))
 (via (at 135.7 85) (size 0.6) (drill 0.3) (layers "F.Cu" "B.Cu") (free yes) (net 2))
 (via (at 125.5 85.4) (size 0.6) (drill 0.3) (layers "F.Cu" "B.Cu") (free yes) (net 2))
 (via (at 123.5 96.1) (size 0.6) (drill 0.3) (layers "F.Cu" "B.Cu") (free yes) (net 2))
 (via (at 130.7 89.1) (size 0.6) (drill 0.3) (layers "F.Cu" "B.Cu") (free yes) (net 2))
 (via (at 134.8 83.1) (size 0.6) (drill 0.3) (layers "F.Cu" "B.Cu") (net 2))
 (via (at 133.9 90.3) (size 0.6) (drill 0.3) (layers "F.Cu" "B.Cu") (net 2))
 (via (at 127.4 95) (size 0.6) (drill 0.3) (layers "F.Cu" "B.Cu") (free yes) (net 2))
 (via (at 130.6 91.4) (size 0.6) (drill 0.3) (layers "F.Cu" "B.Cu") (free yes) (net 2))
 (via (at 135.2 91.6) (size 0.6) (drill 0.3) (layers "F.Cu" "B.Cu") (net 2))
 (via (at 124.7 89.1) (size 0.6) (drill 0.3) (layers "F.Cu" "B.Cu") (free yes) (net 2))
 (via (at 132 87) (size 0.6) (drill 0.3) (layers "F.Cu" "B.Cu") (free yes) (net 2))
 (via (at 127.6 89.9) (size 0.6) (drill 0.3) (layers "F.Cu" "B.Cu") (free yes) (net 2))
 (via (at 135.7 81.5) (size 0.6) (drill 0.3) (layers "F.Cu" "B.Cu") (free yes) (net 2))
 (via (at 124.6 94.5) (size 0.6) (drill 0.3) (layers "F.Cu" "B.Cu") (free yes) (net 2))
 (via (at 132.3 85.6) (size 0.6) (drill 0.3) (layers "F.Cu" "B.Cu") (free yes) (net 2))
 (via (at 129.7 95.1) (size 0.6) (drill 0.3) (layers "F.Cu" "B.Cu") (free yes) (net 2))
 (via (at 128.8 82.8) (size 0.6) (drill 0.3) (layers "F.Cu" "B.Cu") (free yes) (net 2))
 (via (at 130.6 84.3) (size 0.6) (drill 0.3) (layers "F.Cu" "B.Cu") (free yes) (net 2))
 (via (at 123.6 81.4) (size 0.6) (drill 0.3) (layers "F.Cu" "B.Cu") (free yes) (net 2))
 (via (at 130.9 86.7) (size 0.6) (drill 0.3) (layers "F.Cu" "B.Cu") (free yes) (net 2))
 (via (at 127.4 92.1) (size 0.6) (drill 0.3) (layers "F.Cu" "B.Cu") (free yes) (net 2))
 (via (at 135.7 96.15) (size 0.6) (drill 0.3) (layers "F.Cu" "B.Cu") (free yes) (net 2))
 (via (at 130.8 82.1) (size 0.6) (drill 0.3) (layers "F.Cu" "B.Cu") (free yes) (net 2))
 (via (at 128.6 85.4) (size 0.6) (drill 0.3) (layers "F.Cu" "B.Cu") (free yes) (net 2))
 (via (at 129.8 92.1) (size 0.6) (drill 0.3) (layers "F.Cu" "B.Cu") (free yes) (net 2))
 (via (at 124.7 92.4) (size 0.6) (drill 0.3) (layers "F.Cu" "B.Cu") (free yes) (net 2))
 (via (at 125.6 87.8) (size 0.6) (drill 0.3) (layers "F.Cu" "B.Cu") (free yes) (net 2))
 (via (at 133.4 83.5) (size 0.6) (drill 0.3) (layers "F.Cu" "B.Cu") (free yes) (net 2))
 (via (at 128.5 87.7) (size 0.6) (drill 0.3) (layers "F.Cu" "B.Cu") (free yes) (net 2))
 (segment (start 133.4 87.2) (end 133.4 86.7) (width 0.5) (layer "F.Cu") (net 1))
 (segment (start 132 88.6) (end 133.4 87.2) (width 0.5) (layer "F.Cu") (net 1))
 (segment (start 131.975 88.6) (end 132 88.6) (width 0.5) (layer "F.Cu") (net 1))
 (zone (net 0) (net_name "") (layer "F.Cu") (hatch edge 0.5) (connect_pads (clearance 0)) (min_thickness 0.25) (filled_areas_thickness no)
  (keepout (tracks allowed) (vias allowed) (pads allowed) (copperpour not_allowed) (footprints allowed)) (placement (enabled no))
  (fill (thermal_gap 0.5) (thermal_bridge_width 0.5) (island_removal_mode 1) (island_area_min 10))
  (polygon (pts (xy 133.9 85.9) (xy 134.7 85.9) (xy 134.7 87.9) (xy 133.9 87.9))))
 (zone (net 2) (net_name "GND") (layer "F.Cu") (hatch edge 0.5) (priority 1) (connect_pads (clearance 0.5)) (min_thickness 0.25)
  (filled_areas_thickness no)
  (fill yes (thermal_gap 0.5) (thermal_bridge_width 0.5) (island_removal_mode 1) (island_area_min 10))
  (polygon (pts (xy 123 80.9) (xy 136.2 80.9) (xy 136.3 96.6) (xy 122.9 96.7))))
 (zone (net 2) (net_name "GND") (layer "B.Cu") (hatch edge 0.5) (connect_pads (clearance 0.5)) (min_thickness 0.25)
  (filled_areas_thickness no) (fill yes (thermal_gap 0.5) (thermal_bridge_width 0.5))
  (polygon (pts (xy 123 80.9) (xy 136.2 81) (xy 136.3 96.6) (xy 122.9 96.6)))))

